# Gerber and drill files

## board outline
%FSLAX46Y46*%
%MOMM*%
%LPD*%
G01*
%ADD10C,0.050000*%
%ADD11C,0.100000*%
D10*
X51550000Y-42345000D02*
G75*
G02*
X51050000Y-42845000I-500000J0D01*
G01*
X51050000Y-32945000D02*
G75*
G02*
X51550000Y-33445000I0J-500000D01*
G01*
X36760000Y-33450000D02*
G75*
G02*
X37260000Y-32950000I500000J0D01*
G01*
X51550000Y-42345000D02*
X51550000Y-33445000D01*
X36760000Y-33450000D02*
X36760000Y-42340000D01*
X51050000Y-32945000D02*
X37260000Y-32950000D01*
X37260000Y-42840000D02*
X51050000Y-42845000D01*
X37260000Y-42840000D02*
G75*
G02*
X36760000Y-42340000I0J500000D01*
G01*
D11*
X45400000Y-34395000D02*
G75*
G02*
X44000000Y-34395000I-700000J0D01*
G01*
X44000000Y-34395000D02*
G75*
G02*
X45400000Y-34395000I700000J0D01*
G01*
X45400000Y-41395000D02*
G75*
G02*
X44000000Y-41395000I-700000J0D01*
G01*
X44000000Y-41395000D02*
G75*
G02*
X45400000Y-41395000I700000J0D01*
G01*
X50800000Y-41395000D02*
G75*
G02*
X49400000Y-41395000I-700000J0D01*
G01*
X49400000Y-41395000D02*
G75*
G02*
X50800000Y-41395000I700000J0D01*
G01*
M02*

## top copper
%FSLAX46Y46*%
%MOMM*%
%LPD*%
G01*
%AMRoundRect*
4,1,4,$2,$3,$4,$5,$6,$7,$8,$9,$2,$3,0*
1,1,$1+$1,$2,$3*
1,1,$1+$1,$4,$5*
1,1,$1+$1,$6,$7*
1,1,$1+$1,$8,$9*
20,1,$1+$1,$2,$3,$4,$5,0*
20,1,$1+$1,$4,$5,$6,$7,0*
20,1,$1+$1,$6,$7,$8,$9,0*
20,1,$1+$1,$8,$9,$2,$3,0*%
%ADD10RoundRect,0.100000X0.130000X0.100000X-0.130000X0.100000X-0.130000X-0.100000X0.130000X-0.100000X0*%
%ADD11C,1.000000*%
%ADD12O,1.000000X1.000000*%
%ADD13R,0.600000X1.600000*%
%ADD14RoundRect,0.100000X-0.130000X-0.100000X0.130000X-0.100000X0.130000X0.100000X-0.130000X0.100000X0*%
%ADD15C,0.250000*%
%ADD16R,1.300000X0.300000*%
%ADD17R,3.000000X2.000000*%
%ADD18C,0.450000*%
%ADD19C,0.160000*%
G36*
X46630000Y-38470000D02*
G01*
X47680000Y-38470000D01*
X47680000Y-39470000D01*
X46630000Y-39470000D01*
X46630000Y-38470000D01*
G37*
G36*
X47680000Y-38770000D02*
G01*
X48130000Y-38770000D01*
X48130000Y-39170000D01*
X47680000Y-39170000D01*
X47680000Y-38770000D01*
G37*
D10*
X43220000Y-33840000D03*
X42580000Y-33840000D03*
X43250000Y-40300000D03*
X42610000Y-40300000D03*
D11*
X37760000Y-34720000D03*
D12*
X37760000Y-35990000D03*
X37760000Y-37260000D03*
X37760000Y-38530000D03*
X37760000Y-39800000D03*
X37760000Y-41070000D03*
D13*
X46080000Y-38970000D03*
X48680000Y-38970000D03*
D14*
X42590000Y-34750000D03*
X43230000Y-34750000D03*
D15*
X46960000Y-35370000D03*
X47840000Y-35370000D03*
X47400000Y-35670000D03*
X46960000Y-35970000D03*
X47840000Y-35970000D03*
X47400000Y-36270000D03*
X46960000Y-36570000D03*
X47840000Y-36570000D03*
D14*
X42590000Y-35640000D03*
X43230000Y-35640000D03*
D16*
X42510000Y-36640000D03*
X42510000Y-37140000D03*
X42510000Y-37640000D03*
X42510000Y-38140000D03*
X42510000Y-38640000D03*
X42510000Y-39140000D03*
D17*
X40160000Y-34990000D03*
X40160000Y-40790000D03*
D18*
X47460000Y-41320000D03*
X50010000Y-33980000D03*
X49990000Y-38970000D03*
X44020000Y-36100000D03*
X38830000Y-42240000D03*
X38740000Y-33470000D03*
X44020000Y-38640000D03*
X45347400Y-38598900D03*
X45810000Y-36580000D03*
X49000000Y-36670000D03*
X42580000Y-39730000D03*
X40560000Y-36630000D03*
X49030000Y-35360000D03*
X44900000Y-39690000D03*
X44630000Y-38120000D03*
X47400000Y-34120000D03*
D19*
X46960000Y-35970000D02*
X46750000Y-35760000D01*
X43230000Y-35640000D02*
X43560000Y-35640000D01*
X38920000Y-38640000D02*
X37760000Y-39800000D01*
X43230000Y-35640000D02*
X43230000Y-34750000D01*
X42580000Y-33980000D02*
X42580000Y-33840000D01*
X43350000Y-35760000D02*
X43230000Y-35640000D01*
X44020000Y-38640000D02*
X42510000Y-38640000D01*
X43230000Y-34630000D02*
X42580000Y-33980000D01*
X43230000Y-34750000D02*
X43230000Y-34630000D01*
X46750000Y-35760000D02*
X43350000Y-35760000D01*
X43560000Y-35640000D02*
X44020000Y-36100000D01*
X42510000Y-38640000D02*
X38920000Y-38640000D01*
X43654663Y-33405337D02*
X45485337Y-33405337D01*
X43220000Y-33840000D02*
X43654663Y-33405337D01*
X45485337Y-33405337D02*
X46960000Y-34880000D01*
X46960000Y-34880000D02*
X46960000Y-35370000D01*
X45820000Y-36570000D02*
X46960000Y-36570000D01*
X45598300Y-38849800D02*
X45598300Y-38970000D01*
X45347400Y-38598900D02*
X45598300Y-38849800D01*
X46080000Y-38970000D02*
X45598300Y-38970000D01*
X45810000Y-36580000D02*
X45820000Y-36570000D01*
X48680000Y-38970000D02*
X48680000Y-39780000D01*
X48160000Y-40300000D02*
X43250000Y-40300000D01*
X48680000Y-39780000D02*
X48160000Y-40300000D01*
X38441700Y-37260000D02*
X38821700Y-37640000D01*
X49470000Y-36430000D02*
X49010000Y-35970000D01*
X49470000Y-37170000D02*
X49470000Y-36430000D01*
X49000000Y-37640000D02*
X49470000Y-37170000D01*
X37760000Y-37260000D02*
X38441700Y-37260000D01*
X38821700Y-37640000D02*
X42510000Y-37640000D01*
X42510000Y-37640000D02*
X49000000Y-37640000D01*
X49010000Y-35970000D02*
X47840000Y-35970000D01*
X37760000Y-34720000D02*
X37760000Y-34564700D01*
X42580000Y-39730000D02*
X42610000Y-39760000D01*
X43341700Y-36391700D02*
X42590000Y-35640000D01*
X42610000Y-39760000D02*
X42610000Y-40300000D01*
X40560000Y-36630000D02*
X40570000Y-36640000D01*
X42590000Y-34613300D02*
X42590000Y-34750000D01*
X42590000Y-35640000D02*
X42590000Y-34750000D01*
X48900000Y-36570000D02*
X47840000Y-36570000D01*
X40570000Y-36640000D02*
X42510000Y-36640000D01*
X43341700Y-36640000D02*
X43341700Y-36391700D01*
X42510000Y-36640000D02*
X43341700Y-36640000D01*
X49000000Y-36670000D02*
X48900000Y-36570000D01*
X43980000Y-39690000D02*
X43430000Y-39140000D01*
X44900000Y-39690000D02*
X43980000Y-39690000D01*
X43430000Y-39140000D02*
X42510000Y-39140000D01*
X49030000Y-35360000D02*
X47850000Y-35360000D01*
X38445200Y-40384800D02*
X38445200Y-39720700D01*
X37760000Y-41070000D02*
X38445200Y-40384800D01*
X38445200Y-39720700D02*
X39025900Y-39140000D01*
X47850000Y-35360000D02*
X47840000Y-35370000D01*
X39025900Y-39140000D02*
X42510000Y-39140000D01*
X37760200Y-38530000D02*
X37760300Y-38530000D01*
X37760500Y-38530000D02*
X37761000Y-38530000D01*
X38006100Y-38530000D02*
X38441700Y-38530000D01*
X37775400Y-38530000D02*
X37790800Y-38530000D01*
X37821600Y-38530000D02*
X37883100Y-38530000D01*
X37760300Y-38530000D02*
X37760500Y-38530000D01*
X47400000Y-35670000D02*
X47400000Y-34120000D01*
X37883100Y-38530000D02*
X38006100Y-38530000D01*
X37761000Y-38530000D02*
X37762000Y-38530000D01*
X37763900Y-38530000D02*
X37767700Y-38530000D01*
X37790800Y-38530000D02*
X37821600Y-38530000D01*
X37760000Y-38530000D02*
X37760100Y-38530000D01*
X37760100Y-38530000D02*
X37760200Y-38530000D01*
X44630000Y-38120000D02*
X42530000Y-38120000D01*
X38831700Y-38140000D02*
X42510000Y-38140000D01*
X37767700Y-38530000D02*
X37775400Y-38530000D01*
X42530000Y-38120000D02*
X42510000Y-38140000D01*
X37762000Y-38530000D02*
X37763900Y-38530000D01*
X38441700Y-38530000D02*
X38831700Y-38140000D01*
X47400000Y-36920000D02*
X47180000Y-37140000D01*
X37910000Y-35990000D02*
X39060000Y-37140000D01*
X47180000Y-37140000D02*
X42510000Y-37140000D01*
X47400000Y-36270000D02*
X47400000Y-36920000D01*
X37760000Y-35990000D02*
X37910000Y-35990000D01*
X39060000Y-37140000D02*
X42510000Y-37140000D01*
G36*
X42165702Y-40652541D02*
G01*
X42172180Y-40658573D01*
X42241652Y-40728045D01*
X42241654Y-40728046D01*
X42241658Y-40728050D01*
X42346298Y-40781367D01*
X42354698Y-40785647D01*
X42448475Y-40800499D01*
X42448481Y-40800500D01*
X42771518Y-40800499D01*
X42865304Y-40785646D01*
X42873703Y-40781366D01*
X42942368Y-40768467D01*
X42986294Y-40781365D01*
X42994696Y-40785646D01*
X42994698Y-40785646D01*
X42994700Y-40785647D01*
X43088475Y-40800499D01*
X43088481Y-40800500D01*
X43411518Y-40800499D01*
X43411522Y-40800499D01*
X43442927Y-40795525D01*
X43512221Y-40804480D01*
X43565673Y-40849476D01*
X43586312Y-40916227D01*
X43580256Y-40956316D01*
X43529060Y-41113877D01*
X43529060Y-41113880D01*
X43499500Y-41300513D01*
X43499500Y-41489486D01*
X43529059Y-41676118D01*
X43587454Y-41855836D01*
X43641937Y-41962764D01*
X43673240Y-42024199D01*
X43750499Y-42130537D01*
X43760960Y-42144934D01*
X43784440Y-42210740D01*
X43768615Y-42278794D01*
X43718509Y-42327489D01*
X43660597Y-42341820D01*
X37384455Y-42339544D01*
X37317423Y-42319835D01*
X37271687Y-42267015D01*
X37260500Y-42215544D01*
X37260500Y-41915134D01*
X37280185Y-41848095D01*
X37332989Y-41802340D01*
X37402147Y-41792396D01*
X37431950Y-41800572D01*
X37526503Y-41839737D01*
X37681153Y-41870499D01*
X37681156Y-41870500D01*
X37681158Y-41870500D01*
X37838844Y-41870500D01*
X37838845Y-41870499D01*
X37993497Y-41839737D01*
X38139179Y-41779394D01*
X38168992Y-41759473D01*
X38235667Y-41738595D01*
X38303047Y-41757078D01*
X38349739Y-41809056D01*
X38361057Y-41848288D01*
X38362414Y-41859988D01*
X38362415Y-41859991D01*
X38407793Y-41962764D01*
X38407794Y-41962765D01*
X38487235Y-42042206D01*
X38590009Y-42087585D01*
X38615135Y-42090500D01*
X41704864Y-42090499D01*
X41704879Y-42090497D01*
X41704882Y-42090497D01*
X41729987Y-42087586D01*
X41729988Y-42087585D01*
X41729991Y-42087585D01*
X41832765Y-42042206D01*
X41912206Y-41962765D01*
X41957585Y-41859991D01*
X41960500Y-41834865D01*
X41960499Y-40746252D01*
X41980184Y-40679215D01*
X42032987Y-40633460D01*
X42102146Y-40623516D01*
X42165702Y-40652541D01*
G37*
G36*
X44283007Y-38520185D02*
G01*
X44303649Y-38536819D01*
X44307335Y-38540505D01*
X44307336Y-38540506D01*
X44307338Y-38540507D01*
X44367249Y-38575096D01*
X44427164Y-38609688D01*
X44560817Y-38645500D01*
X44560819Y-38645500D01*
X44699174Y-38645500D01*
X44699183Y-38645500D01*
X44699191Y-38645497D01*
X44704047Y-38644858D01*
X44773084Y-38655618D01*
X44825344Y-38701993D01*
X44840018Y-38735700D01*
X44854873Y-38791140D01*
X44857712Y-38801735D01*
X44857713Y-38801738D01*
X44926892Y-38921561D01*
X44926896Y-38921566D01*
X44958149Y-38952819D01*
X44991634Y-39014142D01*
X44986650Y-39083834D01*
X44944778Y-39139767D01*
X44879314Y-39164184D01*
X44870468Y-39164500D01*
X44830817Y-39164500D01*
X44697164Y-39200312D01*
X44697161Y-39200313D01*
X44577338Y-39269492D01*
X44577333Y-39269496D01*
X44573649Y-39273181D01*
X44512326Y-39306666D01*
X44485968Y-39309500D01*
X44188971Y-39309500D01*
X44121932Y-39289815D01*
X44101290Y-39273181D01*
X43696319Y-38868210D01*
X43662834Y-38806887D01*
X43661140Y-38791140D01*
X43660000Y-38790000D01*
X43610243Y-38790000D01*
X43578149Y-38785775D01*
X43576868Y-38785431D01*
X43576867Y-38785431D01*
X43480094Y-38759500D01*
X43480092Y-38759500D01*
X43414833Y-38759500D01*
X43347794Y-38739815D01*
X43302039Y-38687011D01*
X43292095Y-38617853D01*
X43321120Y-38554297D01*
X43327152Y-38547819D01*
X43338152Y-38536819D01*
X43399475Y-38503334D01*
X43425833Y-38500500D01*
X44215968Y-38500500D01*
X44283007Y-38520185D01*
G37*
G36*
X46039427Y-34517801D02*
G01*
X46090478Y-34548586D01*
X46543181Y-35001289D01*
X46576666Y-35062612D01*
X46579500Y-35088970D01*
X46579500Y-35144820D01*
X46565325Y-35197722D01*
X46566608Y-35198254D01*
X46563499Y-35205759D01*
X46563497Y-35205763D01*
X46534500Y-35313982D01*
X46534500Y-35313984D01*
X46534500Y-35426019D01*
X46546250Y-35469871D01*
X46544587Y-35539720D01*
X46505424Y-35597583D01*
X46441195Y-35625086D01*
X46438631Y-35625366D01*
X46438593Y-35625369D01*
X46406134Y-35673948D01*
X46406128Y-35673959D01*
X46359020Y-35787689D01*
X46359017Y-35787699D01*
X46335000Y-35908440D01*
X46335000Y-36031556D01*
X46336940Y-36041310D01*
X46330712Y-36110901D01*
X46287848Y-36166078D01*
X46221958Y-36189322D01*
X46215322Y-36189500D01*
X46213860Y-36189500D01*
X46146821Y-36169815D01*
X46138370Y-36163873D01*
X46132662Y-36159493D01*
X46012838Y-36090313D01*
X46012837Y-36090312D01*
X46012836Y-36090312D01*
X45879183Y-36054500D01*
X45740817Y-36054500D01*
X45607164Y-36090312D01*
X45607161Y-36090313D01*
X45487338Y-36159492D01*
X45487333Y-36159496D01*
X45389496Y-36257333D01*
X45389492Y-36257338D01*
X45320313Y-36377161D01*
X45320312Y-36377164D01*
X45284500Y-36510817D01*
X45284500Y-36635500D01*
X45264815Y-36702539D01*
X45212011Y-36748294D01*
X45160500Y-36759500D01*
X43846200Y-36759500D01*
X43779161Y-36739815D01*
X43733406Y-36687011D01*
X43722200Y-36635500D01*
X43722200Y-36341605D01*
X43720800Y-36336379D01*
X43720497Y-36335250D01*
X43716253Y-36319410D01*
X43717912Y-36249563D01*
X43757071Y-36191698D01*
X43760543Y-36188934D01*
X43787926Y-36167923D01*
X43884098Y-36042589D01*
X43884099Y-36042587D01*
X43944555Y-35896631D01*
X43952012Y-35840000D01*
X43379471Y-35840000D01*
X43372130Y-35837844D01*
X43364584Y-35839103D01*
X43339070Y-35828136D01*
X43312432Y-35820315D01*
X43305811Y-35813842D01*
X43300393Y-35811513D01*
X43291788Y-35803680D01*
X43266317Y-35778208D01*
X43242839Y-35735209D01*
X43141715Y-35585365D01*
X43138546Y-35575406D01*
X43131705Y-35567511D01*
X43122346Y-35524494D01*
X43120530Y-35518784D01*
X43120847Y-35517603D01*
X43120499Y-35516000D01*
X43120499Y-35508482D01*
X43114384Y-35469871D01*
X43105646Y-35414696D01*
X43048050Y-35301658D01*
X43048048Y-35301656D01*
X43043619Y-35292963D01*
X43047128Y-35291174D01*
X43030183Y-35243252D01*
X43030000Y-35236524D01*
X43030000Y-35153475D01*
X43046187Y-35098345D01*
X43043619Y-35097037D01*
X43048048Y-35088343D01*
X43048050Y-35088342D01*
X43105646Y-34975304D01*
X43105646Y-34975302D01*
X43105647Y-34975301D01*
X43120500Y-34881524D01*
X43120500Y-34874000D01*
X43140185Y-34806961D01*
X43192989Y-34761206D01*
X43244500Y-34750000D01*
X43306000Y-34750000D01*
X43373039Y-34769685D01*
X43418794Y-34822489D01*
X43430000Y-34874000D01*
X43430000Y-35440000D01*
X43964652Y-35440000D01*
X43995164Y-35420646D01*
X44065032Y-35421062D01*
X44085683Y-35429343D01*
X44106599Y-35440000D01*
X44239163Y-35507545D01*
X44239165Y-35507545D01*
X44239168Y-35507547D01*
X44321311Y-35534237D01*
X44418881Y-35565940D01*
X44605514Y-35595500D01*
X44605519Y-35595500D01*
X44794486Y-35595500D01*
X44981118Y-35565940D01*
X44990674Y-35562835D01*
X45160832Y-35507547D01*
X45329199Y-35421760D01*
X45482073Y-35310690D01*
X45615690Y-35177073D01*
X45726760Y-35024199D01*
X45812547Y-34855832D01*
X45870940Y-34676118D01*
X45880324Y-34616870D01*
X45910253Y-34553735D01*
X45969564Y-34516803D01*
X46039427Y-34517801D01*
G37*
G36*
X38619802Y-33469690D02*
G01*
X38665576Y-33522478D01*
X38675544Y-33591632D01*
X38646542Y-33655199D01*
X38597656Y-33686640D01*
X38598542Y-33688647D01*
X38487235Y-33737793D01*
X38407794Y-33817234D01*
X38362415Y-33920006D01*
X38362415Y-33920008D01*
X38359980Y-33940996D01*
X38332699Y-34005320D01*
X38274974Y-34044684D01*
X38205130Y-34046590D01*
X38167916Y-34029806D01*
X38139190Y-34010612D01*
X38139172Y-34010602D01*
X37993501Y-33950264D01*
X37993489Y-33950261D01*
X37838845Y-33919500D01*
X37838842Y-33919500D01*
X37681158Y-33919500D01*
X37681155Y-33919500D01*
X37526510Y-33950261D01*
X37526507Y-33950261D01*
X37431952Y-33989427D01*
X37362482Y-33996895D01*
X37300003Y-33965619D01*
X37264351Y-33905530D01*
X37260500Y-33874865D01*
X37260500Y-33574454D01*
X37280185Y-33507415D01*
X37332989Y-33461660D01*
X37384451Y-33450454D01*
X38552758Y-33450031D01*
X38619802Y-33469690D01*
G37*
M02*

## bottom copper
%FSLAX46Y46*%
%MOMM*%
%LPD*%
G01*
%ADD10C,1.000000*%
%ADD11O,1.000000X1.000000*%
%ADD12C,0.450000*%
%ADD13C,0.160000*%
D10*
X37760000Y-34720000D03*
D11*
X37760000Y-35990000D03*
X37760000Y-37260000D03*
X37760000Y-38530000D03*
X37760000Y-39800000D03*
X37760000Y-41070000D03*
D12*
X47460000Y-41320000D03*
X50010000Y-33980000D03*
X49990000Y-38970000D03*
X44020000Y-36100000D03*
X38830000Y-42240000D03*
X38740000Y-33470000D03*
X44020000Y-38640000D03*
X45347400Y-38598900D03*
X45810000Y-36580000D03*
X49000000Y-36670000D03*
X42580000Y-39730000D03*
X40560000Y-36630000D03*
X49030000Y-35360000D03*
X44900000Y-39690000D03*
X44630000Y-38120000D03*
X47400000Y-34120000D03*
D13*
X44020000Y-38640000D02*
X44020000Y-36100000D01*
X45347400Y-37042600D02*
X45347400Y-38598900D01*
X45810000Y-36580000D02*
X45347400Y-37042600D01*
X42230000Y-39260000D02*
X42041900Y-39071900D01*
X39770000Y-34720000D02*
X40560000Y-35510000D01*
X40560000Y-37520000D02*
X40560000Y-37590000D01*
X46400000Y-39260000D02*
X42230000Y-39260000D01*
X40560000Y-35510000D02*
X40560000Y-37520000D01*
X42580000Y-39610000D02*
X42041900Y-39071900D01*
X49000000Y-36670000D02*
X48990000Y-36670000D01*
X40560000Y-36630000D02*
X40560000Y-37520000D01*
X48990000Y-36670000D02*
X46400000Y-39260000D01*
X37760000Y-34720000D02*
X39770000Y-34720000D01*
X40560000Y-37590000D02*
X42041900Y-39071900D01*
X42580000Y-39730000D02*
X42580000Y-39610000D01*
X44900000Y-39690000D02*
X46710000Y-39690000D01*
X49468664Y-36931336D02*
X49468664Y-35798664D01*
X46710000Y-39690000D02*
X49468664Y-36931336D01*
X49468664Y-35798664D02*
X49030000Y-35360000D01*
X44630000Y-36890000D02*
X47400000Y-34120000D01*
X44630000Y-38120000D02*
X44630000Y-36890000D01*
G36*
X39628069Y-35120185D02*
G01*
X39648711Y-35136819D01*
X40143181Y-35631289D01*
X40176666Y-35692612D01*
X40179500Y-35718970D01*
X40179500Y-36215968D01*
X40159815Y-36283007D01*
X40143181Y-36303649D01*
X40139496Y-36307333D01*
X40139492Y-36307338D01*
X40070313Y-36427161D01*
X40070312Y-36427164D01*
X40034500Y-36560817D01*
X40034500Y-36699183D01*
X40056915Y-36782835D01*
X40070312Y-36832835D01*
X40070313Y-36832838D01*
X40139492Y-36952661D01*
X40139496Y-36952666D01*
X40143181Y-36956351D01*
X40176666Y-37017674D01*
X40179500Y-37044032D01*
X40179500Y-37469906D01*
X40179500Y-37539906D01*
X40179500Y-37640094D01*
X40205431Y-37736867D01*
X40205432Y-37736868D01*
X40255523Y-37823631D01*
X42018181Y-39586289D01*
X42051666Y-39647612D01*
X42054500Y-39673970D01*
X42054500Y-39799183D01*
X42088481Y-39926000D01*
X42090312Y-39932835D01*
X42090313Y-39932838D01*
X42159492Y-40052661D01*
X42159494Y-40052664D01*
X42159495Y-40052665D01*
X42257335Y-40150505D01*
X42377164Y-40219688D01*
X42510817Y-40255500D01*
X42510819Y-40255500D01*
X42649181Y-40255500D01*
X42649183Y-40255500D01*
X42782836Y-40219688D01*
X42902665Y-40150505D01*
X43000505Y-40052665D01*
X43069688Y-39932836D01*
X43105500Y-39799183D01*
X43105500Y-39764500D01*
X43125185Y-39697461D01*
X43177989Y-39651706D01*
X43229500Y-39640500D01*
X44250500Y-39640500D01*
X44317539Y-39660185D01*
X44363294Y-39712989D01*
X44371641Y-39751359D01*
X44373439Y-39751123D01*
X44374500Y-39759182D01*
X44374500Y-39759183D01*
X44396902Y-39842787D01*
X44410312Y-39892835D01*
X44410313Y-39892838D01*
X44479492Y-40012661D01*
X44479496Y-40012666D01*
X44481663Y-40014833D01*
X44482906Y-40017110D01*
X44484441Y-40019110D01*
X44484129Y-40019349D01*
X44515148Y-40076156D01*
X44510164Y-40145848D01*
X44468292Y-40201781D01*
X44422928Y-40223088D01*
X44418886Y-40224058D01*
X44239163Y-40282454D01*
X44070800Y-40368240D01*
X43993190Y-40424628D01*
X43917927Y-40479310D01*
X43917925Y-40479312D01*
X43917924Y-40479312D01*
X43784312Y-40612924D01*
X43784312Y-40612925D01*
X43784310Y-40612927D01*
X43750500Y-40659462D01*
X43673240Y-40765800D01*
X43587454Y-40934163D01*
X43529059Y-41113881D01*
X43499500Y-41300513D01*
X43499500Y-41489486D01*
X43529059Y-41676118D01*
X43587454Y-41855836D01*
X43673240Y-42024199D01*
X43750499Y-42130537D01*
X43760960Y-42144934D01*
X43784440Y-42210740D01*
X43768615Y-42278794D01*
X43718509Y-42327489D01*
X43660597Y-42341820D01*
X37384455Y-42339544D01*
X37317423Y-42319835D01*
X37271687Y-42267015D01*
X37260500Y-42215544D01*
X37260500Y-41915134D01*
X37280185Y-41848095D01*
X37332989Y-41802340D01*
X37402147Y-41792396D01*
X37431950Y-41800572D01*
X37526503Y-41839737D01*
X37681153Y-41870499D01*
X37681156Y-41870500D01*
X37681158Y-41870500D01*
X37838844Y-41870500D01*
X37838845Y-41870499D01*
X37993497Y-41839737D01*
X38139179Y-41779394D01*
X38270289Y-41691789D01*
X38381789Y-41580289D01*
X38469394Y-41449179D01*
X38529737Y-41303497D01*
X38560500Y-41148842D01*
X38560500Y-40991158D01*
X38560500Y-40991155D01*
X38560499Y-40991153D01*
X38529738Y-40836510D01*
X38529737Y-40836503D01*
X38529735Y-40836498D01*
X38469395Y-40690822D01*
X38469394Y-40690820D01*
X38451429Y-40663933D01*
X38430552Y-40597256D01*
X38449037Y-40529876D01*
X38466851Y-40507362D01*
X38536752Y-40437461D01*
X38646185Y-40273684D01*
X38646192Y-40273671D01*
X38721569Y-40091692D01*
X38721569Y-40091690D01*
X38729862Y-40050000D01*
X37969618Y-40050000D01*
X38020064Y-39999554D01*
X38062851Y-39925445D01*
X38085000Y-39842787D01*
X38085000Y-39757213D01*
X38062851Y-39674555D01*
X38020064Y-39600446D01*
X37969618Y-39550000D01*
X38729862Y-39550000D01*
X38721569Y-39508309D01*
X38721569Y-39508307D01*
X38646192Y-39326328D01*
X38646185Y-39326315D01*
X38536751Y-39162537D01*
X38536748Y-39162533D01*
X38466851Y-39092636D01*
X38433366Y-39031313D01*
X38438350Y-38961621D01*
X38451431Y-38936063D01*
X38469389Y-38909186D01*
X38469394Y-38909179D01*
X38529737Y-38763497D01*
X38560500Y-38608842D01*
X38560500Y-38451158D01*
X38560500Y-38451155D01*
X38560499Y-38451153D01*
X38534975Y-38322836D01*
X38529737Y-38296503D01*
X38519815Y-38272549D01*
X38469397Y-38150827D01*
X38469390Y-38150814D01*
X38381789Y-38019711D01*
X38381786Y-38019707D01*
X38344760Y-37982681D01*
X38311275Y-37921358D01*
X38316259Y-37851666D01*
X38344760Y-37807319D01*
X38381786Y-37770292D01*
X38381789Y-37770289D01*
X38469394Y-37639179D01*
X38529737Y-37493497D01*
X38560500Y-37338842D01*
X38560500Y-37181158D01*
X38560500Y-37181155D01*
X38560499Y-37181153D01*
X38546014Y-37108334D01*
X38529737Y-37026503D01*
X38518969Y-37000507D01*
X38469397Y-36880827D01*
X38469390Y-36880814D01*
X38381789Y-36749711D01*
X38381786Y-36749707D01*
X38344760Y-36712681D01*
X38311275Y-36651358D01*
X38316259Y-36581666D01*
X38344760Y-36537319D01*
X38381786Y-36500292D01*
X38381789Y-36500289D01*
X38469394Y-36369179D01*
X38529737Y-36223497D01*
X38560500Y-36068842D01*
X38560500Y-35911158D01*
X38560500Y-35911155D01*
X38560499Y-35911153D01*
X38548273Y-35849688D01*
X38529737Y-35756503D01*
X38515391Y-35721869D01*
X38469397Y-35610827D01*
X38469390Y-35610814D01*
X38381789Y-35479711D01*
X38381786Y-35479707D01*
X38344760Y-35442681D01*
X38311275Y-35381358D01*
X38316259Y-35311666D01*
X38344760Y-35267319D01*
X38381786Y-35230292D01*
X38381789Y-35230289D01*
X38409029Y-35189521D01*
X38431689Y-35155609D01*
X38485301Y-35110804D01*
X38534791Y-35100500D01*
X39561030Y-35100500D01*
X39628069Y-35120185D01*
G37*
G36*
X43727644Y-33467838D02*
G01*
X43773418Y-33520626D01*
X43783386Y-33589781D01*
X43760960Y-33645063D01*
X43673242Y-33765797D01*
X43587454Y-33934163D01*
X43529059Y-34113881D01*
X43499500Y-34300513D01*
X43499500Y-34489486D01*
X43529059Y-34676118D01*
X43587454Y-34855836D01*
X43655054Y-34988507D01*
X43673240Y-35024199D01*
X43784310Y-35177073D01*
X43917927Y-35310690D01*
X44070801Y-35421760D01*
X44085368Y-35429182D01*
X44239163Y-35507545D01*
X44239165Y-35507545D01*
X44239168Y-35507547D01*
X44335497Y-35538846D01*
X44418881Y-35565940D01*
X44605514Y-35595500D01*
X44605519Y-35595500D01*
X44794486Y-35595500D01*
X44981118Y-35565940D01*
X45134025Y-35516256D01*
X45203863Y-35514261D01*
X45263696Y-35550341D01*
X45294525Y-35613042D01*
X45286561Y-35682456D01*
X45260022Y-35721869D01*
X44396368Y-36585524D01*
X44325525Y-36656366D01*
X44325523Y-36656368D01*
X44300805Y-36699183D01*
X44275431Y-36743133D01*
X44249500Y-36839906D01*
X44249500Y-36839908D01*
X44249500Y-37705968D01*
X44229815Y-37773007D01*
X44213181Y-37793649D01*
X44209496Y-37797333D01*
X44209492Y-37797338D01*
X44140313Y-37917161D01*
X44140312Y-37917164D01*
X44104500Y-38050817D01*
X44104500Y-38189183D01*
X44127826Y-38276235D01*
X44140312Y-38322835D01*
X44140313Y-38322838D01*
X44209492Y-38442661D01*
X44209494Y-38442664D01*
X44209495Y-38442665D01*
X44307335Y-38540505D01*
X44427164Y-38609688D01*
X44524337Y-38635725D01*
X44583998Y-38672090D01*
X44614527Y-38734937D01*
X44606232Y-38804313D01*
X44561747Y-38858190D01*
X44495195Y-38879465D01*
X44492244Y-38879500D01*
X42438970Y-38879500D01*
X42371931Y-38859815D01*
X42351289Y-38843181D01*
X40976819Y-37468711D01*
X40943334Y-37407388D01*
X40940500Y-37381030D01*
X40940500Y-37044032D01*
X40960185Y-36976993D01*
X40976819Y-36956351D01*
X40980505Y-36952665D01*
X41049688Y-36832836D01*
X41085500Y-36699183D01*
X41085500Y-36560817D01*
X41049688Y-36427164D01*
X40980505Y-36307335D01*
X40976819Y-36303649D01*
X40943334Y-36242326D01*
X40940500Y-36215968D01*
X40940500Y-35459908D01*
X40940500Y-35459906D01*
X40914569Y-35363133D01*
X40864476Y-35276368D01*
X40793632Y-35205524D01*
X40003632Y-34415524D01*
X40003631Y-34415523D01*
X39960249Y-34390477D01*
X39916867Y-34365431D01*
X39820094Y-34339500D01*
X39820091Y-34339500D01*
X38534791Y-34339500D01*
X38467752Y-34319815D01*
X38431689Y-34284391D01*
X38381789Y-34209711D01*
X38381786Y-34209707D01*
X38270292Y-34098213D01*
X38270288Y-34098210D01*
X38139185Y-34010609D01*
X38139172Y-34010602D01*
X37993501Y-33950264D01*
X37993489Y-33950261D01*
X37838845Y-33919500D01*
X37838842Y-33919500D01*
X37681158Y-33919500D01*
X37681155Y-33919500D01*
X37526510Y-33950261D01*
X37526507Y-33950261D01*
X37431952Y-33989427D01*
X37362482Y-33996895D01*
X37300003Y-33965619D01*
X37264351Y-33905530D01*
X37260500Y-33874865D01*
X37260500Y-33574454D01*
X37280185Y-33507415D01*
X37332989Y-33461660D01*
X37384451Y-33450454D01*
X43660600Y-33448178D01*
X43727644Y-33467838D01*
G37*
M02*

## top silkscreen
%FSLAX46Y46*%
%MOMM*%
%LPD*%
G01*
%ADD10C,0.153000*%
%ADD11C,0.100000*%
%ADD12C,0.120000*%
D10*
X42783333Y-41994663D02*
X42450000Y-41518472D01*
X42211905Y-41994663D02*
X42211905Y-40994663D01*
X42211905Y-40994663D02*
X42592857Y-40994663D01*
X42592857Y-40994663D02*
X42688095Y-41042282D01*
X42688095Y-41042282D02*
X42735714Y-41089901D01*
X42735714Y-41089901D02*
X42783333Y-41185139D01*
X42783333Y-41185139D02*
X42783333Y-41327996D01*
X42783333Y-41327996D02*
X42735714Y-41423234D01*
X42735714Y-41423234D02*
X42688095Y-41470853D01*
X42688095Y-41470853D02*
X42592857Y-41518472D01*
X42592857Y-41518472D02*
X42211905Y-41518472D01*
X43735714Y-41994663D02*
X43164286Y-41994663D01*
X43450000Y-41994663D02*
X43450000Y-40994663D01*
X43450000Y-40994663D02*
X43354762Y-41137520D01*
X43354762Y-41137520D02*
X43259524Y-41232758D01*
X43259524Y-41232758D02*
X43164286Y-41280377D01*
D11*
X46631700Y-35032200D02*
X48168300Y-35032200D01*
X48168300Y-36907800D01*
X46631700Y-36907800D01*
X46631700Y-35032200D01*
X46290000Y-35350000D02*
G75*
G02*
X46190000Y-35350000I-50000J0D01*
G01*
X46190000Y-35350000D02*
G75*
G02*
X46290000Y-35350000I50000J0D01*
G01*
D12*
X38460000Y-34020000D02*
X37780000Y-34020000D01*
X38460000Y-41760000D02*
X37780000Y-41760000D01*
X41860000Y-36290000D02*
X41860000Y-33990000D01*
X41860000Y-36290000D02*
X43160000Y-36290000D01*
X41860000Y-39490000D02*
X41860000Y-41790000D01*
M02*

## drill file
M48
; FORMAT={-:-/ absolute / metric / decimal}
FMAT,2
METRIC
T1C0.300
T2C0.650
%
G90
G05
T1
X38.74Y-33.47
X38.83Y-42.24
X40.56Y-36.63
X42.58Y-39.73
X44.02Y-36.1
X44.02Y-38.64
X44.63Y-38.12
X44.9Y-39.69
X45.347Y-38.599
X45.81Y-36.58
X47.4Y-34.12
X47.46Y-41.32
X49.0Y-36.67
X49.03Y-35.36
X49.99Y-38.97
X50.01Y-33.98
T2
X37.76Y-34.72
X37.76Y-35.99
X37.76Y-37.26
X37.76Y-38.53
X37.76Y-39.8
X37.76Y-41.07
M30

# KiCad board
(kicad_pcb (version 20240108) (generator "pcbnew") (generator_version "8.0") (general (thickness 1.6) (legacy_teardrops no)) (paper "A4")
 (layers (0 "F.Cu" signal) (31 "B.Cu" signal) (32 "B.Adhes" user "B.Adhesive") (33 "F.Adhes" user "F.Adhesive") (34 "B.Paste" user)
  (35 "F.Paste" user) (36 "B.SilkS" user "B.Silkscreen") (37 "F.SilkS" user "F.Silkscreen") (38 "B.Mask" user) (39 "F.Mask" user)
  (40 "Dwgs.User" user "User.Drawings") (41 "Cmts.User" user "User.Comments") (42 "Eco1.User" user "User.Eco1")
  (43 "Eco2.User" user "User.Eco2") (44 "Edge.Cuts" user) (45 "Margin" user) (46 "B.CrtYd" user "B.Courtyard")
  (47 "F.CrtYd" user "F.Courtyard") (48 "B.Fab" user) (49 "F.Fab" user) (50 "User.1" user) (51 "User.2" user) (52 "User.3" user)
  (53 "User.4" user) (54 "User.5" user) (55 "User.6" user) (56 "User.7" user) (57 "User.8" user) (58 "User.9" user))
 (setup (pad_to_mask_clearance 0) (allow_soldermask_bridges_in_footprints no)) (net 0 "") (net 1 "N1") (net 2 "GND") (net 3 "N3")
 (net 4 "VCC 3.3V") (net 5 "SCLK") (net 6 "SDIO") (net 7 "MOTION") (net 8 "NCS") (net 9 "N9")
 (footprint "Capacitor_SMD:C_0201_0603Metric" (layer "F.Cu") (at 42.9 33.84 180)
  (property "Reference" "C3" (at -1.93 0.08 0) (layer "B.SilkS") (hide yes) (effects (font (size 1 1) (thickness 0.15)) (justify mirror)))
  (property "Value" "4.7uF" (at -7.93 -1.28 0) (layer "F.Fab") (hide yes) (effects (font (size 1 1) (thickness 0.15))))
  (pad "" smd roundrect (at -0.345 0 180) (size 0.318 0.36) (layers "F.Paste") (roundrect_rratio 0.25))
  (pad "" smd roundrect (at 0.345 0 180) (size 0.318 0.36) (layers "F.Paste") (roundrect_rratio 0.25))
  (pad "1" smd roundrect (at -0.32 0 180) (size 0.46 0.4) (layers "F.Cu" "F.Mask") (roundrect_rratio 0.25) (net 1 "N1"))
  (pad "2" smd roundrect (at 0.32 0 180) (size 0.46 0.4) (layers "F.Cu" "F.Mask") (roundrect_rratio 0.25) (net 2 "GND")))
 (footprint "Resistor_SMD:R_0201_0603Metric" (layer "F.Cu") (at 42.93 40.3 180)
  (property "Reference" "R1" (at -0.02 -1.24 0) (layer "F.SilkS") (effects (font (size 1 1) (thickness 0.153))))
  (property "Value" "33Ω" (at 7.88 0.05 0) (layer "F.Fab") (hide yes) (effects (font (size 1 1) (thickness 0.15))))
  (pad "" smd roundrect (at -0.345 0 180) (size 0.318 0.36) (layers "F.Paste") (roundrect_rratio 0.25))
  (pad "" smd roundrect (at 0.345 0 180) (size 0.318 0.36) (layers "F.Paste") (roundrect_rratio 0.25))
  (pad "1" smd roundrect (at -0.32 0 180) (size 0.46 0.4) (layers "F.Cu" "F.Mask") (roundrect_rratio 0.25) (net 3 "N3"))
  (pad "2" smd roundrect (at 0.32 0 180) (size 0.46 0.4) (layers "F.Cu" "F.Mask") (roundrect_rratio 0.25) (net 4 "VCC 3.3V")))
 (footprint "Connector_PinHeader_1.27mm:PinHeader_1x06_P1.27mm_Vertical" (layer "F.Cu") (at 37.76 34.72)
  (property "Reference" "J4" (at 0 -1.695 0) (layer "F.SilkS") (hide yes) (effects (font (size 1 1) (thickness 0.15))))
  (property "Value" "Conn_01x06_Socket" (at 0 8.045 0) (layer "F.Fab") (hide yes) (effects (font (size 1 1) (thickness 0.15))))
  (pad "1" thru_hole circle (at 0 0) (size 1 1) (drill 0.65) (layers "*.Cu" "*.Mask") (remove_unused_layers no) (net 4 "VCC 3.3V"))
  (pad "2" thru_hole oval (at 0 1.27) (size 1 1) (drill 0.65) (layers "*.Cu" "*.Mask") (remove_unused_layers no) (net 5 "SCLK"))
  (pad "3" thru_hole oval (at 0 2.54) (size 1 1) (drill 0.65) (layers "*.Cu" "*.Mask") (remove_unused_layers no) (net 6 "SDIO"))
  (pad "4" thru_hole oval (at 0 3.81) (size 1 1) (drill 0.65) (layers "*.Cu" "*.Mask") (remove_unused_layers no) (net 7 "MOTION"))
  (pad "5" thru_hole oval (at 0 5.08) (size 1 1) (drill 0.65) (layers "*.Cu" "*.Mask") (remove_unused_layers no) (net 2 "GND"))
  (pad "6" thru_hole oval (at 0 6.35) (size 1 1) (drill 0.65) (layers "*.Cu" "*.Mask") (remove_unused_layers no) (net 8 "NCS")))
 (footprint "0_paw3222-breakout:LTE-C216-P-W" (layer "F.Cu") (at 47.38 38.97 90)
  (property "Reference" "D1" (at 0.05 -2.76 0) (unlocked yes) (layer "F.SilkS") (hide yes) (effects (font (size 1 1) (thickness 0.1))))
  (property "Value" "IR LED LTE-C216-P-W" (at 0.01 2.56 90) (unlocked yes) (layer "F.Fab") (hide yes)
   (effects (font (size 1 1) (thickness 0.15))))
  (fp_rect (start -0.5 -0.75) (end 0.5 0.3) (stroke (width 0) (type solid)) (fill solid) (layer "F.Cu"))
  (fp_rect (start -0.2 0.3) (end 0.2 0.75) (stroke (width 0) (type solid)) (fill solid) (layer "F.Cu"))
  (pad "1" smd rect (at 0 -1.3 90) (size 1.6 0.6) (layers "F.Cu" "F.Paste" "F.Mask") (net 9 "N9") (thermal_bridge_angle 45))
  (pad "2" smd rect (at 0 1.3 90) (size 1.6 0.6) (layers "F.Cu" "F.Paste" "F.Mask") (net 3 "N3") (thermal_bridge_angle 45)))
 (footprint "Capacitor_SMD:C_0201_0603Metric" (layer "F.Cu") (at 42.91 34.75)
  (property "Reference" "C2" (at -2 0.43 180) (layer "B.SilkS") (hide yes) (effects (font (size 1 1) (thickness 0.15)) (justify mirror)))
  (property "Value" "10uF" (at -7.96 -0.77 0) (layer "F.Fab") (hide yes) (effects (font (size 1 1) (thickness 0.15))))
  (pad "" smd roundrect (at -0.345 0) (size 0.318 0.36) (layers "F.Paste") (roundrect_rratio 0.25))
  (pad "" smd roundrect (at 0.345 0) (size 0.318 0.36) (layers "F.Paste") (roundrect_rratio 0.25))
  (pad "1" smd roundrect (at -0.32 0) (size 0.46 0.4) (layers "F.Cu" "F.Mask") (roundrect_rratio 0.25) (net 4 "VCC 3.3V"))
  (pad "2" smd roundrect (at 0.32 0) (size 0.46 0.4) (layers "F.Cu" "F.Mask") (roundrect_rratio 0.25) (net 2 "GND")))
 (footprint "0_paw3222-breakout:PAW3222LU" (layer "F.Cu") (at 47.4 35.97)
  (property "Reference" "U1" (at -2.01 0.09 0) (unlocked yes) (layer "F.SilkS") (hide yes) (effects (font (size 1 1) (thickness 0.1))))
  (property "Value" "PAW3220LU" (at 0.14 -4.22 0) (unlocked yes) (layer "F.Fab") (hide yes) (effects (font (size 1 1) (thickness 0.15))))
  (fp_rect (start -0.7683 -0.9378) (end 0.7683 0.9378) (stroke (width 0.1) (type default)) (fill none) (layer "F.SilkS"))
  (fp_circle (center -1.16 -0.62) (end -1.06 -0.62) (stroke (width 0) (type solid)) (fill solid) (layer "F.SilkS"))
  (fp_circle (center -2.7 -1.575) (end -2 -1.575) (stroke (width 0.1) (type default)) (fill none) (layer "Edge.Cuts"))
  (fp_circle (center -2.7 5.425) (end -2 5.425) (stroke (width 0.1) (type default)) (fill none) (layer "Edge.Cuts"))
  (fp_circle (center 2.7 5.425) (end 3.4 5.425) (stroke (width 0.1) (type default)) (fill none) (layer "Edge.Cuts"))
  (pad "A1" smd circle (at -0.44 -0.6) (size 0.25 0.25) (layers "F.Cu" "F.Paste" "F.Mask") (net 1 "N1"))
  (pad "A3" smd circle (at 0.44 -0.6) (size 0.25 0.25) (layers "F.Cu" "F.Paste" "F.Mask") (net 8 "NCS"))
  (pad "B2" smd circle (at 0 -0.3) (size 0.25 0.25) (layers "F.Cu" "F.Paste" "F.Mask") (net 7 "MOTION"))
  (pad "C1" smd circle (at -0.44 0) (size 0.25 0.25) (layers "F.Cu" "F.Paste" "F.Mask") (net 2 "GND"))
  (pad "C3" smd circle (at 0.44 0) (size 0.25 0.25) (layers "F.Cu" "F.Paste" "F.Mask") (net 6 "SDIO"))
  (pad "D2" smd circle (at 0 0.3) (size 0.25 0.25) (layers "F.Cu" "F.Paste" "F.Mask") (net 5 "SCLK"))
  (pad "E1" smd circle (at -0.44 0.6) (size 0.25 0.25) (layers "F.Cu" "F.Paste" "F.Mask") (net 9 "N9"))
  (pad "E3" smd circle (at 0.44 0.6) (size 0.25 0.25) (layers "F.Cu" "F.Paste" "F.Mask") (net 4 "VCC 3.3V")))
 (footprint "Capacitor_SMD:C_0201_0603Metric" (layer "F.Cu") (at 42.91 35.64)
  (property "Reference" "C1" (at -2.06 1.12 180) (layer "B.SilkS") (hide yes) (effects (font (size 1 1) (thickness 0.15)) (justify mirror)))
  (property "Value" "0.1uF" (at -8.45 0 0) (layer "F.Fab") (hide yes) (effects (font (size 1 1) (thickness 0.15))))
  (pad "" smd roundrect (at -0.345 0) (size 0.318 0.36) (layers "F.Paste") (roundrect_rratio 0.25))
  (pad "" smd roundrect (at 0.345 0) (size 0.318 0.36) (layers "F.Paste") (roundrect_rratio 0.25))
  (pad "1" smd roundrect (at -0.32 0) (size 0.46 0.4) (layers "F.Cu" "F.Mask") (roundrect_rratio 0.25) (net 4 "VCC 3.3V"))
  (pad "2" smd roundrect (at 0.32 0) (size 0.46 0.4) (layers "F.Cu" "F.Mask") (roundrect_rratio 0.25) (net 2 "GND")))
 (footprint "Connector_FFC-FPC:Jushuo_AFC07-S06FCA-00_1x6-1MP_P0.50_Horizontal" (layer "F.Cu") (at 40.91 37.89 -90)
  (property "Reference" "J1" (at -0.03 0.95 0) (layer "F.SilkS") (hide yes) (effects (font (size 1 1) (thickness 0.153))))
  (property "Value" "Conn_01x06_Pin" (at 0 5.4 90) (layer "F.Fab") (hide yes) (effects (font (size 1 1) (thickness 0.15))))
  (fp_line (start -3.87 2.45) (end -3.87 3.13) (stroke (width 0.12) (type solid)) (layer "F.SilkS"))
  (fp_line (start 3.87 2.45) (end 3.87 3.13) (stroke (width 0.12) (type solid)) (layer "F.SilkS"))
  (fp_line (start -1.6 -0.95) (end -3.9 -0.95) (stroke (width 0.12) (type solid)) (layer "F.SilkS"))
  (fp_line (start -1.6 -0.95) (end -1.6 -2.25) (stroke (width 0.12) (type solid)) (layer "F.SilkS"))
  (fp_line (start 1.6 -0.95) (end 3.9 -0.95) (stroke (width 0.12) (type solid)) (layer "F.SilkS"))
  (pad "1" smd rect (at -1.25 -1.6 270) (size 0.3 1.3) (layers "F.Cu" "F.Paste" "F.Mask") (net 4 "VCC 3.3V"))
  (pad "2" smd rect (at -0.75 -1.6 270) (size 0.3 1.3) (layers "F.Cu" "F.Paste" "F.Mask") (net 5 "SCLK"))
  (pad "3" smd rect (at -0.25 -1.6 270) (size 0.3 1.3) (layers "F.Cu" "F.Paste" "F.Mask") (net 6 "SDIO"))
  (pad "4" smd rect (at 0.25 -1.6 270) (size 0.3 1.3) (layers "F.Cu" "F.Paste" "F.Mask") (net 7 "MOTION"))
  (pad "5" smd rect (at 0.75 -1.6 270) (size 0.3 1.3) (layers "F.Cu" "F.Paste" "F.Mask") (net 2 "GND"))
  (pad "6" smd rect (at 1.25 -1.6 270) (size 0.3 1.3) (layers "F.Cu" "F.Paste" "F.Mask") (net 8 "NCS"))
  (pad "MP" smd rect (at -2.9 0.75 270) (size 2 3) (layers "F.Cu" "F.Paste" "F.Mask"))
  (pad "MP" smd rect (at 2.9 0.75 270) (size 2 3) (layers "F.Cu" "F.Paste" "F.Mask")))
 (gr_arc (start 51.55 42.345) (mid 51.403553 42.698553) (end 51.05 42.845) (stroke (width 0.05) (type default)) (layer "Edge.Cuts"))
 (gr_arc (start 51.05 32.945) (mid 51.403553 33.091447) (end 51.55 33.445) (stroke (width 0.05) (type default)) (layer "Edge.Cuts"))
 (gr_arc (start 36.76 33.45) (mid 36.906447 33.096447) (end 37.26 32.95) (stroke (width 0.05) (type default)) (layer "Edge.Cuts"))
 (gr_line (start 51.55 42.345) (end 51.55 33.445) (stroke (width 0.05) (type default)) (layer "Edge.Cuts"))
 (gr_line (start 36.76 33.45) (end 36.76 42.34) (stroke (width 0.05) (type default)) (layer "Edge.Cuts"))
 (gr_line (start 51.05 32.945) (end 37.26 32.95) (stroke (width 0.05) (type default)) (layer "Edge.Cuts"))
 (gr_line (start 37.26 42.84) (end 51.05 42.845) (stroke (width 0.05) (type default)) (layer "Edge.Cuts"))
 (gr_arc (start 37.26 42.84) (mid 36.906447 42.693553) (end 36.76 42.34) (stroke (width 0.05) (type default)) (layer "Edge.Cuts"))
 (segment (start 46.96 35.97) (end 46.75 35.76) (width 0.16) (layer "F.Cu") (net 2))
 (segment (start 43.23 35.64) (end 43.56 35.64) (width 0.16) (layer "F.Cu") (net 2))
 (segment (start 38.92 38.64) (end 37.76 39.8) (width 0.16) (layer "F.Cu") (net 2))
 (segment (start 43.23 35.64) (end 43.23 34.75) (width 0.16) (layer "F.Cu") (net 2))
 (segment (start 42.58 33.98) (end 42.58 33.84) (width 0.16) (layer "F.Cu") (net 2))
 (segment (start 43.35 35.76) (end 43.23 35.64) (width 0.16) (layer "F.Cu") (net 2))
 (segment (start 44.02 38.64) (end 42.51 38.64) (width 0.16) (layer "F.Cu") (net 2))
 (segment (start 43.23 34.63) (end 42.58 33.98) (width 0.16) (layer "F.Cu") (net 2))
 (segment (start 43.23 34.75) (end 43.23 34.63) (width 0.16) (layer "F.Cu") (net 2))
 (segment (start 46.75 35.76) (end 43.35 35.76) (width 0.16) (layer "F.Cu") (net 2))
 (segment (start 43.56 35.64) (end 44.02 36.1) (width 0.16) (layer "F.Cu") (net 2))
 (segment (start 42.51 38.64) (end 38.92 38.64) (width 0.16) (layer "F.Cu") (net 2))
 (via micro (at 47.46 41.32) (size 0.45) (drill 0.3) (layers "F.Cu" "B.Cu") (free yes) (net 2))
 (via micro (at 50.01 33.98) (size 0.45) (drill 0.3) (layers "F.Cu" "B.Cu") (free yes) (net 2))
 (via micro (at 49.99 38.97) (size 0.45) (drill 0.3) (layers "F.Cu" "B.Cu") (free yes) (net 2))
 (via micro (at 44.02 36.1) (size 0.45) (drill 0.3) (layers "F.Cu" "B.Cu") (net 2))
 (via micro (at 38.83 42.24) (size 0.45) (drill 0.3) (layers "F.Cu" "B.Cu") (free yes) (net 2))
 (via micro (at 38.74 33.47) (size 0.45) (drill 0.3) (layers "F.Cu" "B.Cu") (free yes) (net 2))
 (via micro (at 44.02 38.64) (size 0.45) (drill 0.3) (layers "F.Cu" "B.Cu") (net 2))
 (segment (start 44.02 38.64) (end 44.02 36.1) (width 0.16) (layer "B.Cu") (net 2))
 (segment (start 43.654663 33.405337) (end 45.485337 33.405337) (width 0.16) (layer "F.Cu") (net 1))
 (segment (start 43.22 33.84) (end 43.654663 33.405337) (width 0.16) (layer "F.Cu") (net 1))
 (segment (start 45.485337 33.405337) (end 46.96 34.88) (width 0.16) (layer "F.Cu") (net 1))
 (segment (start 46.96 34.88) (end 46.96 35.37) (width 0.16) (layer "F.Cu") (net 1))
 (segment (start 45.82 36.57) (end 46.96 36.57) (width 0.16) (layer "F.Cu") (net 9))
 (segment (start 45.5983 38.8498) (end 45.5983 38.97) (width 0.16) (layer "F.Cu") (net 9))
 (segment (start 45.3474 38.5989) (end 45.5983 38.8498) (width 0.16) (layer "F.Cu") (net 9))
 (segment (start 46.08 38.97) (end 45.5983 38.97) (width 0.16) (layer "F.Cu") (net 9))
 (segment (start 45.81 36.58) (end 45.82 36.57) (width 0.16) (layer "F.Cu") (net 9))
 (via micro (at 45.3474 38.5989) (size 0.45) (drill 0.3) (layers "F.Cu" "B.Cu") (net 9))
 (via micro (at 45.81 36.58) (size 0.45) (drill 0.3) (layers "F.Cu" "B.Cu") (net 9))
 (segment (start 45.3474 37.0426) (end 45.3474 38.5989) (width 0.16) (layer "B.Cu") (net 9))
 (segment (start 45.81 36.58) (end 45.3474 37.0426) (width 0.16) (layer "B.Cu") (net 9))
 (segment (start 48.68 38.97) (end 48.68 39.78) (width 0.16) (layer "F.Cu") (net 3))
 (segment (start 48.16 40.3) (end 43.25 40.3) (width 0.16) (layer "F.Cu") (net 3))
 (segment (start 48.68 39.78) (end 48.16 40.3) (width 0.16) (layer "F.Cu") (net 3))
 (segment (start 38.4417 37.26) (end 38.8217 37.64) (width 0.16) (layer "F.Cu") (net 6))
 (segment (start 49.47 36.43) (end 49.01 35.97) (width 0.16) (layer "F.Cu") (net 6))
 (segment (start 49.47 37.17) (end 49.47 36.43) (width 0.16) (layer "F.Cu") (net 6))
 (segment (start 49 37.64) (end 49.47 37.17) (width 0.16) (layer "F.Cu") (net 6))
 (segment (start 37.76 37.26) (end 38.4417 37.26) (width 0.16) (layer "F.Cu") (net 6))
 (segment (start 38.8217 37.64) (end 42.51 37.64) (width 0.16) (layer "F.Cu") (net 6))
 (segment (start 42.51 37.64) (end 49 37.64) (width 0.16) (layer "F.Cu") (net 6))
 (segment (start 49.01 35.97) (end 47.84 35.97) (width 0.16) (layer "F.Cu") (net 6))
 (segment (start 37.76 34.72) (end 37.76 34.5647) (width 0.16) (layer "F.Cu") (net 4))
 (segment (start 42.58 39.73) (end 42.61 39.76) (width 0.16) (layer "F.Cu") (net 4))
 (segment (start 43.3417 36.3917) (end 42.59 35.64) (width 0.16) (layer "F.Cu") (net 4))
 (segment (start 42.61 39.76) (end 42.61 40.3) (width 0.16) (layer "F.Cu") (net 4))
 (segment (start 40.56 36.63) (end 40.57 36.64) (width 0.16) (layer "F.Cu") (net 4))
 (segment (start 42.59 34.6133) (end 42.59 34.75) (width 0.16) (layer "F.Cu") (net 4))
 (segment (start 42.59 35.64) (end 42.59 34.75) (width 0.16) (layer "F.Cu") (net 4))
 (segment (start 48.9 36.57) (end 47.84 36.57) (width 0.16) (layer "F.Cu") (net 4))
 (segment (start 40.57 36.64) (end 42.51 36.64) (width 0.16) (layer "F.Cu") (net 4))
 (segment (start 43.3417 36.64) (end 43.3417 36.3917) (width 0.16) (layer "F.Cu") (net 4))
 (segment (start 42.51 36.64) (end 43.3417 36.64) (width 0.16) (layer "F.Cu") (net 4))
 (segment (start 49 36.67) (end 48.9 36.57) (width 0.16) (layer "F.Cu") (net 4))
 (via micro (at 49 36.67) (size 0.45) (drill 0.3) (layers "F.Cu" "B.Cu") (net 4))
 (via micro (at 42.58 39.73) (size 0.45) (drill 0.3) (layers "F.Cu" "B.Cu") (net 4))
 (via micro (at 40.56 36.63) (size 0.45) (drill 0.3) (layers "F.Cu" "B.Cu") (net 4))
 (segment (start 42.23 39.26) (end 42.0419 39.0719) (width 0.16) (layer "B.Cu") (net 4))
 (segment (start 39.77 34.72) (end 40.56 35.51) (width 0.16) (layer "B.Cu") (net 4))
 (segment (start 40.56 37.52) (end 40.56 37.59) (width 0.16) (layer "B.Cu") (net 4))
 (segment (start 46.4 39.26) (end 42.23 39.26) (width 0.16) (layer "B.Cu") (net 4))
 (segment (start 40.56 35.51) (end 40.56 37.52) (width 0.16) (layer "B.Cu") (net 4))
 (segment (start 42.58 39.61) (end 42.0419 39.0719) (width 0.16) (layer "B.Cu") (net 4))
 (segment (start 49 36.67) (end 48.99 36.67) (width 0.16) (layer "B.Cu") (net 4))
 (segment (start 40.56 36.63) (end 40.56 37.52) (width 0.16) (layer "B.Cu") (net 4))
 (segment (start 48.99 36.67) (end 46.4 39.26) (width 0.16) (layer "B.Cu") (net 4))
 (segment (start 37.76 34.72) (end 39.77 34.72) (width 0.16) (layer "B.Cu") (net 4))
 (segment (start 40.56 37.59) (end 42.0419 39.0719) (width 0.16) (layer "B.Cu") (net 4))
 (segment (start 42.58 39.73) (end 42.58 39.61) (width 0.16) (layer "B.Cu") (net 4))
 (segment (start 43.98 39.69) (end 43.43 39.14) (width 0.16) (layer "F.Cu") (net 8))
 (segment (start 44.9 39.69) (end 43.98 39.69) (width 0.16) (layer "F.Cu") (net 8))
 (segment (start 43.43 39.14) (end 42.51 39.14) (width 0.16) (layer "F.Cu") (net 8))
 (segment (start 49.03 35.36) (end 47.85 35.36) (width 0.16) (layer "F.Cu") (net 8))
 (segment (start 38.4452 40.3848) (end 38.4452 39.7207) (width 0.16) (layer "F.Cu") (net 8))
 (segment (start 37.76 41.07) (end 38.4452 40.3848) (width 0.16) (layer "F.Cu") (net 8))
 (segment (start 38.4452 39.7207) (end 39.0259 39.14) (width 0.16) (layer "F.Cu") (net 8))
 (segment (start 47.85 35.36) (end 47.84 35.37) (width 0.16) (layer "F.Cu") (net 8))
 (segment (start 39.0259 39.14) (end 42.51 39.14) (width 0.16) (layer "F.Cu") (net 8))
 (via micro (at 49.03 35.36) (size 0.45) (drill 0.3) (layers "F.Cu" "B.Cu") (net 8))
 (via micro (at 44.9 39.69) (size 0.45) (drill 0.3) (layers "F.Cu" "B.Cu") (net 8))
 (segment (start 44.9 39.69) (end 46.71 39.69) (width 0.16) (layer "B.Cu") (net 8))
 (segment (start 49.468664 36.931336) (end 49.468664 35.798664) (width 0.16) (layer "B.Cu") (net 8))
 (segment (start 46.71 39.69) (end 49.468664 36.931336) (width 0.16) (layer "B.Cu") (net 8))
 (segment (start 49.468664 35.798664) (end 49.03 35.36) (width 0.16) (layer "B.Cu") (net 8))
 (segment (start 37.7602 38.53) (end 37.7603 38.53) (width 0.16) (layer "F.Cu") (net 7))
 (segment (start 37.7605 38.53) (end 37.761 38.53) (width 0.16) (layer "F.Cu") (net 7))
 (segment (start 38.0061 38.53) (end 38.4417 38.53) (width 0.16) (layer "F.Cu") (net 7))
 (segment (start 37.7754 38.53) (end 37.7908 38.53) (width 0.16) (layer "F.Cu") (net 7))
 (segment (start 37.8216 38.53) (end 37.8831 38.53) (width 0.16) (layer "F.Cu") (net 7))
 (segment (start 37.7603 38.53) (end 37.7605 38.53) (width 0.16) (layer "F.Cu") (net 7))
 (segment (start 47.4 35.67) (end 47.4 34.12) (width 0.16) (layer "F.Cu") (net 7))
 (segment (start 37.8831 38.53) (end 38.0061 38.53) (width 0.16) (layer "F.Cu") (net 7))
 (segment (start 37.761 38.53) (end 37.762 38.53) (width 0.16) (layer "F.Cu") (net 7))
 (segment (start 37.7639 38.53) (end 37.7677 38.53) (width 0.16) (layer "F.Cu") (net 7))
 (segment (start 37.7908 38.53) (end 37.8216 38.53) (width 0.16) (layer "F.Cu") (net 7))
 (segment (start 37.76 38.53) (end 37.7601 38.53) (width 0.16) (layer "F.Cu") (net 7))
 (segment (start 37.7601 38.53) (end 37.7602 38.53) (width 0.16) (layer "F.Cu") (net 7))
 (segment (start 44.63 38.12) (end 42.53 38.12) (width 0.16) (layer "F.Cu") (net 7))
 (segment (start 38.8317 38.14) (end 42.51 38.14) (width 0.16) (layer "F.Cu") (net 7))
 (segment (start 37.7677 38.53) (end 37.7754 38.53) (width 0.16) (layer "F.Cu") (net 7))
 (segment (start 42.53 38.12) (end 42.51 38.14) (width 0.16) (layer "F.Cu") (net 7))
 (segment (start 37.762 38.53) (end 37.7639 38.53) (width 0.16) (layer "F.Cu") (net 7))
 (segment (start 38.4417 38.53) (end 38.8317 38.14) (width 0.16) (layer "F.Cu") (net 7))
 (via micro (at 44.63 38.12) (size 0.45) (drill 0.3) (layers "F.Cu" "B.Cu") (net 7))
 (via micro (at 47.4 34.12) (size 0.45) (drill 0.3) (layers "F.Cu" "B.Cu") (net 7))
 (segment (start 44.63 36.89) (end 47.4 34.12) (width 0.16) (layer "B.Cu") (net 7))
 (segment (start 44.63 38.12) (end 44.63 36.89) (width 0.16) (layer "B.Cu") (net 7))
 (segment (start 47.4 36.92) (end 47.18 37.14) (width 0.16) (layer "F.Cu") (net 5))
 (segment (start 37.91 35.99) (end 39.06 37.14) (width 0.16) (layer "F.Cu") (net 5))
 (segment (start 47.18 37.14) (end 42.51 37.14) (width 0.16) (layer "F.Cu") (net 5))
 (segment (start 47.4 36.27) (end 47.4 36.92) (width 0.16) (layer "F.Cu") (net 5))
 (segment (start 37.76 35.99) (end 37.91 35.99) (width 0.16) (layer "F.Cu") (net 5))
 (segment (start 39.06 37.14) (end 42.51 37.14) (width 0.16) (layer "F.Cu") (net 5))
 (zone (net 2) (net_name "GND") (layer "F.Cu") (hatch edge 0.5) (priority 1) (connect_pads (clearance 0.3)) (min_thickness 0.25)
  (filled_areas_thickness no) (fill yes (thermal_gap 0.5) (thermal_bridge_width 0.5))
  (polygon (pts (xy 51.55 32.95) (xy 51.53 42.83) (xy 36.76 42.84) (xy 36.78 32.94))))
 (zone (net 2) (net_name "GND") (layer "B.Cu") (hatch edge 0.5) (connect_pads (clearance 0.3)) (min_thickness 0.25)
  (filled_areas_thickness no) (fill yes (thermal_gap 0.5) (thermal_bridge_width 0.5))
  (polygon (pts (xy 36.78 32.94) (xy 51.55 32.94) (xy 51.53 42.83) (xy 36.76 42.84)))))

